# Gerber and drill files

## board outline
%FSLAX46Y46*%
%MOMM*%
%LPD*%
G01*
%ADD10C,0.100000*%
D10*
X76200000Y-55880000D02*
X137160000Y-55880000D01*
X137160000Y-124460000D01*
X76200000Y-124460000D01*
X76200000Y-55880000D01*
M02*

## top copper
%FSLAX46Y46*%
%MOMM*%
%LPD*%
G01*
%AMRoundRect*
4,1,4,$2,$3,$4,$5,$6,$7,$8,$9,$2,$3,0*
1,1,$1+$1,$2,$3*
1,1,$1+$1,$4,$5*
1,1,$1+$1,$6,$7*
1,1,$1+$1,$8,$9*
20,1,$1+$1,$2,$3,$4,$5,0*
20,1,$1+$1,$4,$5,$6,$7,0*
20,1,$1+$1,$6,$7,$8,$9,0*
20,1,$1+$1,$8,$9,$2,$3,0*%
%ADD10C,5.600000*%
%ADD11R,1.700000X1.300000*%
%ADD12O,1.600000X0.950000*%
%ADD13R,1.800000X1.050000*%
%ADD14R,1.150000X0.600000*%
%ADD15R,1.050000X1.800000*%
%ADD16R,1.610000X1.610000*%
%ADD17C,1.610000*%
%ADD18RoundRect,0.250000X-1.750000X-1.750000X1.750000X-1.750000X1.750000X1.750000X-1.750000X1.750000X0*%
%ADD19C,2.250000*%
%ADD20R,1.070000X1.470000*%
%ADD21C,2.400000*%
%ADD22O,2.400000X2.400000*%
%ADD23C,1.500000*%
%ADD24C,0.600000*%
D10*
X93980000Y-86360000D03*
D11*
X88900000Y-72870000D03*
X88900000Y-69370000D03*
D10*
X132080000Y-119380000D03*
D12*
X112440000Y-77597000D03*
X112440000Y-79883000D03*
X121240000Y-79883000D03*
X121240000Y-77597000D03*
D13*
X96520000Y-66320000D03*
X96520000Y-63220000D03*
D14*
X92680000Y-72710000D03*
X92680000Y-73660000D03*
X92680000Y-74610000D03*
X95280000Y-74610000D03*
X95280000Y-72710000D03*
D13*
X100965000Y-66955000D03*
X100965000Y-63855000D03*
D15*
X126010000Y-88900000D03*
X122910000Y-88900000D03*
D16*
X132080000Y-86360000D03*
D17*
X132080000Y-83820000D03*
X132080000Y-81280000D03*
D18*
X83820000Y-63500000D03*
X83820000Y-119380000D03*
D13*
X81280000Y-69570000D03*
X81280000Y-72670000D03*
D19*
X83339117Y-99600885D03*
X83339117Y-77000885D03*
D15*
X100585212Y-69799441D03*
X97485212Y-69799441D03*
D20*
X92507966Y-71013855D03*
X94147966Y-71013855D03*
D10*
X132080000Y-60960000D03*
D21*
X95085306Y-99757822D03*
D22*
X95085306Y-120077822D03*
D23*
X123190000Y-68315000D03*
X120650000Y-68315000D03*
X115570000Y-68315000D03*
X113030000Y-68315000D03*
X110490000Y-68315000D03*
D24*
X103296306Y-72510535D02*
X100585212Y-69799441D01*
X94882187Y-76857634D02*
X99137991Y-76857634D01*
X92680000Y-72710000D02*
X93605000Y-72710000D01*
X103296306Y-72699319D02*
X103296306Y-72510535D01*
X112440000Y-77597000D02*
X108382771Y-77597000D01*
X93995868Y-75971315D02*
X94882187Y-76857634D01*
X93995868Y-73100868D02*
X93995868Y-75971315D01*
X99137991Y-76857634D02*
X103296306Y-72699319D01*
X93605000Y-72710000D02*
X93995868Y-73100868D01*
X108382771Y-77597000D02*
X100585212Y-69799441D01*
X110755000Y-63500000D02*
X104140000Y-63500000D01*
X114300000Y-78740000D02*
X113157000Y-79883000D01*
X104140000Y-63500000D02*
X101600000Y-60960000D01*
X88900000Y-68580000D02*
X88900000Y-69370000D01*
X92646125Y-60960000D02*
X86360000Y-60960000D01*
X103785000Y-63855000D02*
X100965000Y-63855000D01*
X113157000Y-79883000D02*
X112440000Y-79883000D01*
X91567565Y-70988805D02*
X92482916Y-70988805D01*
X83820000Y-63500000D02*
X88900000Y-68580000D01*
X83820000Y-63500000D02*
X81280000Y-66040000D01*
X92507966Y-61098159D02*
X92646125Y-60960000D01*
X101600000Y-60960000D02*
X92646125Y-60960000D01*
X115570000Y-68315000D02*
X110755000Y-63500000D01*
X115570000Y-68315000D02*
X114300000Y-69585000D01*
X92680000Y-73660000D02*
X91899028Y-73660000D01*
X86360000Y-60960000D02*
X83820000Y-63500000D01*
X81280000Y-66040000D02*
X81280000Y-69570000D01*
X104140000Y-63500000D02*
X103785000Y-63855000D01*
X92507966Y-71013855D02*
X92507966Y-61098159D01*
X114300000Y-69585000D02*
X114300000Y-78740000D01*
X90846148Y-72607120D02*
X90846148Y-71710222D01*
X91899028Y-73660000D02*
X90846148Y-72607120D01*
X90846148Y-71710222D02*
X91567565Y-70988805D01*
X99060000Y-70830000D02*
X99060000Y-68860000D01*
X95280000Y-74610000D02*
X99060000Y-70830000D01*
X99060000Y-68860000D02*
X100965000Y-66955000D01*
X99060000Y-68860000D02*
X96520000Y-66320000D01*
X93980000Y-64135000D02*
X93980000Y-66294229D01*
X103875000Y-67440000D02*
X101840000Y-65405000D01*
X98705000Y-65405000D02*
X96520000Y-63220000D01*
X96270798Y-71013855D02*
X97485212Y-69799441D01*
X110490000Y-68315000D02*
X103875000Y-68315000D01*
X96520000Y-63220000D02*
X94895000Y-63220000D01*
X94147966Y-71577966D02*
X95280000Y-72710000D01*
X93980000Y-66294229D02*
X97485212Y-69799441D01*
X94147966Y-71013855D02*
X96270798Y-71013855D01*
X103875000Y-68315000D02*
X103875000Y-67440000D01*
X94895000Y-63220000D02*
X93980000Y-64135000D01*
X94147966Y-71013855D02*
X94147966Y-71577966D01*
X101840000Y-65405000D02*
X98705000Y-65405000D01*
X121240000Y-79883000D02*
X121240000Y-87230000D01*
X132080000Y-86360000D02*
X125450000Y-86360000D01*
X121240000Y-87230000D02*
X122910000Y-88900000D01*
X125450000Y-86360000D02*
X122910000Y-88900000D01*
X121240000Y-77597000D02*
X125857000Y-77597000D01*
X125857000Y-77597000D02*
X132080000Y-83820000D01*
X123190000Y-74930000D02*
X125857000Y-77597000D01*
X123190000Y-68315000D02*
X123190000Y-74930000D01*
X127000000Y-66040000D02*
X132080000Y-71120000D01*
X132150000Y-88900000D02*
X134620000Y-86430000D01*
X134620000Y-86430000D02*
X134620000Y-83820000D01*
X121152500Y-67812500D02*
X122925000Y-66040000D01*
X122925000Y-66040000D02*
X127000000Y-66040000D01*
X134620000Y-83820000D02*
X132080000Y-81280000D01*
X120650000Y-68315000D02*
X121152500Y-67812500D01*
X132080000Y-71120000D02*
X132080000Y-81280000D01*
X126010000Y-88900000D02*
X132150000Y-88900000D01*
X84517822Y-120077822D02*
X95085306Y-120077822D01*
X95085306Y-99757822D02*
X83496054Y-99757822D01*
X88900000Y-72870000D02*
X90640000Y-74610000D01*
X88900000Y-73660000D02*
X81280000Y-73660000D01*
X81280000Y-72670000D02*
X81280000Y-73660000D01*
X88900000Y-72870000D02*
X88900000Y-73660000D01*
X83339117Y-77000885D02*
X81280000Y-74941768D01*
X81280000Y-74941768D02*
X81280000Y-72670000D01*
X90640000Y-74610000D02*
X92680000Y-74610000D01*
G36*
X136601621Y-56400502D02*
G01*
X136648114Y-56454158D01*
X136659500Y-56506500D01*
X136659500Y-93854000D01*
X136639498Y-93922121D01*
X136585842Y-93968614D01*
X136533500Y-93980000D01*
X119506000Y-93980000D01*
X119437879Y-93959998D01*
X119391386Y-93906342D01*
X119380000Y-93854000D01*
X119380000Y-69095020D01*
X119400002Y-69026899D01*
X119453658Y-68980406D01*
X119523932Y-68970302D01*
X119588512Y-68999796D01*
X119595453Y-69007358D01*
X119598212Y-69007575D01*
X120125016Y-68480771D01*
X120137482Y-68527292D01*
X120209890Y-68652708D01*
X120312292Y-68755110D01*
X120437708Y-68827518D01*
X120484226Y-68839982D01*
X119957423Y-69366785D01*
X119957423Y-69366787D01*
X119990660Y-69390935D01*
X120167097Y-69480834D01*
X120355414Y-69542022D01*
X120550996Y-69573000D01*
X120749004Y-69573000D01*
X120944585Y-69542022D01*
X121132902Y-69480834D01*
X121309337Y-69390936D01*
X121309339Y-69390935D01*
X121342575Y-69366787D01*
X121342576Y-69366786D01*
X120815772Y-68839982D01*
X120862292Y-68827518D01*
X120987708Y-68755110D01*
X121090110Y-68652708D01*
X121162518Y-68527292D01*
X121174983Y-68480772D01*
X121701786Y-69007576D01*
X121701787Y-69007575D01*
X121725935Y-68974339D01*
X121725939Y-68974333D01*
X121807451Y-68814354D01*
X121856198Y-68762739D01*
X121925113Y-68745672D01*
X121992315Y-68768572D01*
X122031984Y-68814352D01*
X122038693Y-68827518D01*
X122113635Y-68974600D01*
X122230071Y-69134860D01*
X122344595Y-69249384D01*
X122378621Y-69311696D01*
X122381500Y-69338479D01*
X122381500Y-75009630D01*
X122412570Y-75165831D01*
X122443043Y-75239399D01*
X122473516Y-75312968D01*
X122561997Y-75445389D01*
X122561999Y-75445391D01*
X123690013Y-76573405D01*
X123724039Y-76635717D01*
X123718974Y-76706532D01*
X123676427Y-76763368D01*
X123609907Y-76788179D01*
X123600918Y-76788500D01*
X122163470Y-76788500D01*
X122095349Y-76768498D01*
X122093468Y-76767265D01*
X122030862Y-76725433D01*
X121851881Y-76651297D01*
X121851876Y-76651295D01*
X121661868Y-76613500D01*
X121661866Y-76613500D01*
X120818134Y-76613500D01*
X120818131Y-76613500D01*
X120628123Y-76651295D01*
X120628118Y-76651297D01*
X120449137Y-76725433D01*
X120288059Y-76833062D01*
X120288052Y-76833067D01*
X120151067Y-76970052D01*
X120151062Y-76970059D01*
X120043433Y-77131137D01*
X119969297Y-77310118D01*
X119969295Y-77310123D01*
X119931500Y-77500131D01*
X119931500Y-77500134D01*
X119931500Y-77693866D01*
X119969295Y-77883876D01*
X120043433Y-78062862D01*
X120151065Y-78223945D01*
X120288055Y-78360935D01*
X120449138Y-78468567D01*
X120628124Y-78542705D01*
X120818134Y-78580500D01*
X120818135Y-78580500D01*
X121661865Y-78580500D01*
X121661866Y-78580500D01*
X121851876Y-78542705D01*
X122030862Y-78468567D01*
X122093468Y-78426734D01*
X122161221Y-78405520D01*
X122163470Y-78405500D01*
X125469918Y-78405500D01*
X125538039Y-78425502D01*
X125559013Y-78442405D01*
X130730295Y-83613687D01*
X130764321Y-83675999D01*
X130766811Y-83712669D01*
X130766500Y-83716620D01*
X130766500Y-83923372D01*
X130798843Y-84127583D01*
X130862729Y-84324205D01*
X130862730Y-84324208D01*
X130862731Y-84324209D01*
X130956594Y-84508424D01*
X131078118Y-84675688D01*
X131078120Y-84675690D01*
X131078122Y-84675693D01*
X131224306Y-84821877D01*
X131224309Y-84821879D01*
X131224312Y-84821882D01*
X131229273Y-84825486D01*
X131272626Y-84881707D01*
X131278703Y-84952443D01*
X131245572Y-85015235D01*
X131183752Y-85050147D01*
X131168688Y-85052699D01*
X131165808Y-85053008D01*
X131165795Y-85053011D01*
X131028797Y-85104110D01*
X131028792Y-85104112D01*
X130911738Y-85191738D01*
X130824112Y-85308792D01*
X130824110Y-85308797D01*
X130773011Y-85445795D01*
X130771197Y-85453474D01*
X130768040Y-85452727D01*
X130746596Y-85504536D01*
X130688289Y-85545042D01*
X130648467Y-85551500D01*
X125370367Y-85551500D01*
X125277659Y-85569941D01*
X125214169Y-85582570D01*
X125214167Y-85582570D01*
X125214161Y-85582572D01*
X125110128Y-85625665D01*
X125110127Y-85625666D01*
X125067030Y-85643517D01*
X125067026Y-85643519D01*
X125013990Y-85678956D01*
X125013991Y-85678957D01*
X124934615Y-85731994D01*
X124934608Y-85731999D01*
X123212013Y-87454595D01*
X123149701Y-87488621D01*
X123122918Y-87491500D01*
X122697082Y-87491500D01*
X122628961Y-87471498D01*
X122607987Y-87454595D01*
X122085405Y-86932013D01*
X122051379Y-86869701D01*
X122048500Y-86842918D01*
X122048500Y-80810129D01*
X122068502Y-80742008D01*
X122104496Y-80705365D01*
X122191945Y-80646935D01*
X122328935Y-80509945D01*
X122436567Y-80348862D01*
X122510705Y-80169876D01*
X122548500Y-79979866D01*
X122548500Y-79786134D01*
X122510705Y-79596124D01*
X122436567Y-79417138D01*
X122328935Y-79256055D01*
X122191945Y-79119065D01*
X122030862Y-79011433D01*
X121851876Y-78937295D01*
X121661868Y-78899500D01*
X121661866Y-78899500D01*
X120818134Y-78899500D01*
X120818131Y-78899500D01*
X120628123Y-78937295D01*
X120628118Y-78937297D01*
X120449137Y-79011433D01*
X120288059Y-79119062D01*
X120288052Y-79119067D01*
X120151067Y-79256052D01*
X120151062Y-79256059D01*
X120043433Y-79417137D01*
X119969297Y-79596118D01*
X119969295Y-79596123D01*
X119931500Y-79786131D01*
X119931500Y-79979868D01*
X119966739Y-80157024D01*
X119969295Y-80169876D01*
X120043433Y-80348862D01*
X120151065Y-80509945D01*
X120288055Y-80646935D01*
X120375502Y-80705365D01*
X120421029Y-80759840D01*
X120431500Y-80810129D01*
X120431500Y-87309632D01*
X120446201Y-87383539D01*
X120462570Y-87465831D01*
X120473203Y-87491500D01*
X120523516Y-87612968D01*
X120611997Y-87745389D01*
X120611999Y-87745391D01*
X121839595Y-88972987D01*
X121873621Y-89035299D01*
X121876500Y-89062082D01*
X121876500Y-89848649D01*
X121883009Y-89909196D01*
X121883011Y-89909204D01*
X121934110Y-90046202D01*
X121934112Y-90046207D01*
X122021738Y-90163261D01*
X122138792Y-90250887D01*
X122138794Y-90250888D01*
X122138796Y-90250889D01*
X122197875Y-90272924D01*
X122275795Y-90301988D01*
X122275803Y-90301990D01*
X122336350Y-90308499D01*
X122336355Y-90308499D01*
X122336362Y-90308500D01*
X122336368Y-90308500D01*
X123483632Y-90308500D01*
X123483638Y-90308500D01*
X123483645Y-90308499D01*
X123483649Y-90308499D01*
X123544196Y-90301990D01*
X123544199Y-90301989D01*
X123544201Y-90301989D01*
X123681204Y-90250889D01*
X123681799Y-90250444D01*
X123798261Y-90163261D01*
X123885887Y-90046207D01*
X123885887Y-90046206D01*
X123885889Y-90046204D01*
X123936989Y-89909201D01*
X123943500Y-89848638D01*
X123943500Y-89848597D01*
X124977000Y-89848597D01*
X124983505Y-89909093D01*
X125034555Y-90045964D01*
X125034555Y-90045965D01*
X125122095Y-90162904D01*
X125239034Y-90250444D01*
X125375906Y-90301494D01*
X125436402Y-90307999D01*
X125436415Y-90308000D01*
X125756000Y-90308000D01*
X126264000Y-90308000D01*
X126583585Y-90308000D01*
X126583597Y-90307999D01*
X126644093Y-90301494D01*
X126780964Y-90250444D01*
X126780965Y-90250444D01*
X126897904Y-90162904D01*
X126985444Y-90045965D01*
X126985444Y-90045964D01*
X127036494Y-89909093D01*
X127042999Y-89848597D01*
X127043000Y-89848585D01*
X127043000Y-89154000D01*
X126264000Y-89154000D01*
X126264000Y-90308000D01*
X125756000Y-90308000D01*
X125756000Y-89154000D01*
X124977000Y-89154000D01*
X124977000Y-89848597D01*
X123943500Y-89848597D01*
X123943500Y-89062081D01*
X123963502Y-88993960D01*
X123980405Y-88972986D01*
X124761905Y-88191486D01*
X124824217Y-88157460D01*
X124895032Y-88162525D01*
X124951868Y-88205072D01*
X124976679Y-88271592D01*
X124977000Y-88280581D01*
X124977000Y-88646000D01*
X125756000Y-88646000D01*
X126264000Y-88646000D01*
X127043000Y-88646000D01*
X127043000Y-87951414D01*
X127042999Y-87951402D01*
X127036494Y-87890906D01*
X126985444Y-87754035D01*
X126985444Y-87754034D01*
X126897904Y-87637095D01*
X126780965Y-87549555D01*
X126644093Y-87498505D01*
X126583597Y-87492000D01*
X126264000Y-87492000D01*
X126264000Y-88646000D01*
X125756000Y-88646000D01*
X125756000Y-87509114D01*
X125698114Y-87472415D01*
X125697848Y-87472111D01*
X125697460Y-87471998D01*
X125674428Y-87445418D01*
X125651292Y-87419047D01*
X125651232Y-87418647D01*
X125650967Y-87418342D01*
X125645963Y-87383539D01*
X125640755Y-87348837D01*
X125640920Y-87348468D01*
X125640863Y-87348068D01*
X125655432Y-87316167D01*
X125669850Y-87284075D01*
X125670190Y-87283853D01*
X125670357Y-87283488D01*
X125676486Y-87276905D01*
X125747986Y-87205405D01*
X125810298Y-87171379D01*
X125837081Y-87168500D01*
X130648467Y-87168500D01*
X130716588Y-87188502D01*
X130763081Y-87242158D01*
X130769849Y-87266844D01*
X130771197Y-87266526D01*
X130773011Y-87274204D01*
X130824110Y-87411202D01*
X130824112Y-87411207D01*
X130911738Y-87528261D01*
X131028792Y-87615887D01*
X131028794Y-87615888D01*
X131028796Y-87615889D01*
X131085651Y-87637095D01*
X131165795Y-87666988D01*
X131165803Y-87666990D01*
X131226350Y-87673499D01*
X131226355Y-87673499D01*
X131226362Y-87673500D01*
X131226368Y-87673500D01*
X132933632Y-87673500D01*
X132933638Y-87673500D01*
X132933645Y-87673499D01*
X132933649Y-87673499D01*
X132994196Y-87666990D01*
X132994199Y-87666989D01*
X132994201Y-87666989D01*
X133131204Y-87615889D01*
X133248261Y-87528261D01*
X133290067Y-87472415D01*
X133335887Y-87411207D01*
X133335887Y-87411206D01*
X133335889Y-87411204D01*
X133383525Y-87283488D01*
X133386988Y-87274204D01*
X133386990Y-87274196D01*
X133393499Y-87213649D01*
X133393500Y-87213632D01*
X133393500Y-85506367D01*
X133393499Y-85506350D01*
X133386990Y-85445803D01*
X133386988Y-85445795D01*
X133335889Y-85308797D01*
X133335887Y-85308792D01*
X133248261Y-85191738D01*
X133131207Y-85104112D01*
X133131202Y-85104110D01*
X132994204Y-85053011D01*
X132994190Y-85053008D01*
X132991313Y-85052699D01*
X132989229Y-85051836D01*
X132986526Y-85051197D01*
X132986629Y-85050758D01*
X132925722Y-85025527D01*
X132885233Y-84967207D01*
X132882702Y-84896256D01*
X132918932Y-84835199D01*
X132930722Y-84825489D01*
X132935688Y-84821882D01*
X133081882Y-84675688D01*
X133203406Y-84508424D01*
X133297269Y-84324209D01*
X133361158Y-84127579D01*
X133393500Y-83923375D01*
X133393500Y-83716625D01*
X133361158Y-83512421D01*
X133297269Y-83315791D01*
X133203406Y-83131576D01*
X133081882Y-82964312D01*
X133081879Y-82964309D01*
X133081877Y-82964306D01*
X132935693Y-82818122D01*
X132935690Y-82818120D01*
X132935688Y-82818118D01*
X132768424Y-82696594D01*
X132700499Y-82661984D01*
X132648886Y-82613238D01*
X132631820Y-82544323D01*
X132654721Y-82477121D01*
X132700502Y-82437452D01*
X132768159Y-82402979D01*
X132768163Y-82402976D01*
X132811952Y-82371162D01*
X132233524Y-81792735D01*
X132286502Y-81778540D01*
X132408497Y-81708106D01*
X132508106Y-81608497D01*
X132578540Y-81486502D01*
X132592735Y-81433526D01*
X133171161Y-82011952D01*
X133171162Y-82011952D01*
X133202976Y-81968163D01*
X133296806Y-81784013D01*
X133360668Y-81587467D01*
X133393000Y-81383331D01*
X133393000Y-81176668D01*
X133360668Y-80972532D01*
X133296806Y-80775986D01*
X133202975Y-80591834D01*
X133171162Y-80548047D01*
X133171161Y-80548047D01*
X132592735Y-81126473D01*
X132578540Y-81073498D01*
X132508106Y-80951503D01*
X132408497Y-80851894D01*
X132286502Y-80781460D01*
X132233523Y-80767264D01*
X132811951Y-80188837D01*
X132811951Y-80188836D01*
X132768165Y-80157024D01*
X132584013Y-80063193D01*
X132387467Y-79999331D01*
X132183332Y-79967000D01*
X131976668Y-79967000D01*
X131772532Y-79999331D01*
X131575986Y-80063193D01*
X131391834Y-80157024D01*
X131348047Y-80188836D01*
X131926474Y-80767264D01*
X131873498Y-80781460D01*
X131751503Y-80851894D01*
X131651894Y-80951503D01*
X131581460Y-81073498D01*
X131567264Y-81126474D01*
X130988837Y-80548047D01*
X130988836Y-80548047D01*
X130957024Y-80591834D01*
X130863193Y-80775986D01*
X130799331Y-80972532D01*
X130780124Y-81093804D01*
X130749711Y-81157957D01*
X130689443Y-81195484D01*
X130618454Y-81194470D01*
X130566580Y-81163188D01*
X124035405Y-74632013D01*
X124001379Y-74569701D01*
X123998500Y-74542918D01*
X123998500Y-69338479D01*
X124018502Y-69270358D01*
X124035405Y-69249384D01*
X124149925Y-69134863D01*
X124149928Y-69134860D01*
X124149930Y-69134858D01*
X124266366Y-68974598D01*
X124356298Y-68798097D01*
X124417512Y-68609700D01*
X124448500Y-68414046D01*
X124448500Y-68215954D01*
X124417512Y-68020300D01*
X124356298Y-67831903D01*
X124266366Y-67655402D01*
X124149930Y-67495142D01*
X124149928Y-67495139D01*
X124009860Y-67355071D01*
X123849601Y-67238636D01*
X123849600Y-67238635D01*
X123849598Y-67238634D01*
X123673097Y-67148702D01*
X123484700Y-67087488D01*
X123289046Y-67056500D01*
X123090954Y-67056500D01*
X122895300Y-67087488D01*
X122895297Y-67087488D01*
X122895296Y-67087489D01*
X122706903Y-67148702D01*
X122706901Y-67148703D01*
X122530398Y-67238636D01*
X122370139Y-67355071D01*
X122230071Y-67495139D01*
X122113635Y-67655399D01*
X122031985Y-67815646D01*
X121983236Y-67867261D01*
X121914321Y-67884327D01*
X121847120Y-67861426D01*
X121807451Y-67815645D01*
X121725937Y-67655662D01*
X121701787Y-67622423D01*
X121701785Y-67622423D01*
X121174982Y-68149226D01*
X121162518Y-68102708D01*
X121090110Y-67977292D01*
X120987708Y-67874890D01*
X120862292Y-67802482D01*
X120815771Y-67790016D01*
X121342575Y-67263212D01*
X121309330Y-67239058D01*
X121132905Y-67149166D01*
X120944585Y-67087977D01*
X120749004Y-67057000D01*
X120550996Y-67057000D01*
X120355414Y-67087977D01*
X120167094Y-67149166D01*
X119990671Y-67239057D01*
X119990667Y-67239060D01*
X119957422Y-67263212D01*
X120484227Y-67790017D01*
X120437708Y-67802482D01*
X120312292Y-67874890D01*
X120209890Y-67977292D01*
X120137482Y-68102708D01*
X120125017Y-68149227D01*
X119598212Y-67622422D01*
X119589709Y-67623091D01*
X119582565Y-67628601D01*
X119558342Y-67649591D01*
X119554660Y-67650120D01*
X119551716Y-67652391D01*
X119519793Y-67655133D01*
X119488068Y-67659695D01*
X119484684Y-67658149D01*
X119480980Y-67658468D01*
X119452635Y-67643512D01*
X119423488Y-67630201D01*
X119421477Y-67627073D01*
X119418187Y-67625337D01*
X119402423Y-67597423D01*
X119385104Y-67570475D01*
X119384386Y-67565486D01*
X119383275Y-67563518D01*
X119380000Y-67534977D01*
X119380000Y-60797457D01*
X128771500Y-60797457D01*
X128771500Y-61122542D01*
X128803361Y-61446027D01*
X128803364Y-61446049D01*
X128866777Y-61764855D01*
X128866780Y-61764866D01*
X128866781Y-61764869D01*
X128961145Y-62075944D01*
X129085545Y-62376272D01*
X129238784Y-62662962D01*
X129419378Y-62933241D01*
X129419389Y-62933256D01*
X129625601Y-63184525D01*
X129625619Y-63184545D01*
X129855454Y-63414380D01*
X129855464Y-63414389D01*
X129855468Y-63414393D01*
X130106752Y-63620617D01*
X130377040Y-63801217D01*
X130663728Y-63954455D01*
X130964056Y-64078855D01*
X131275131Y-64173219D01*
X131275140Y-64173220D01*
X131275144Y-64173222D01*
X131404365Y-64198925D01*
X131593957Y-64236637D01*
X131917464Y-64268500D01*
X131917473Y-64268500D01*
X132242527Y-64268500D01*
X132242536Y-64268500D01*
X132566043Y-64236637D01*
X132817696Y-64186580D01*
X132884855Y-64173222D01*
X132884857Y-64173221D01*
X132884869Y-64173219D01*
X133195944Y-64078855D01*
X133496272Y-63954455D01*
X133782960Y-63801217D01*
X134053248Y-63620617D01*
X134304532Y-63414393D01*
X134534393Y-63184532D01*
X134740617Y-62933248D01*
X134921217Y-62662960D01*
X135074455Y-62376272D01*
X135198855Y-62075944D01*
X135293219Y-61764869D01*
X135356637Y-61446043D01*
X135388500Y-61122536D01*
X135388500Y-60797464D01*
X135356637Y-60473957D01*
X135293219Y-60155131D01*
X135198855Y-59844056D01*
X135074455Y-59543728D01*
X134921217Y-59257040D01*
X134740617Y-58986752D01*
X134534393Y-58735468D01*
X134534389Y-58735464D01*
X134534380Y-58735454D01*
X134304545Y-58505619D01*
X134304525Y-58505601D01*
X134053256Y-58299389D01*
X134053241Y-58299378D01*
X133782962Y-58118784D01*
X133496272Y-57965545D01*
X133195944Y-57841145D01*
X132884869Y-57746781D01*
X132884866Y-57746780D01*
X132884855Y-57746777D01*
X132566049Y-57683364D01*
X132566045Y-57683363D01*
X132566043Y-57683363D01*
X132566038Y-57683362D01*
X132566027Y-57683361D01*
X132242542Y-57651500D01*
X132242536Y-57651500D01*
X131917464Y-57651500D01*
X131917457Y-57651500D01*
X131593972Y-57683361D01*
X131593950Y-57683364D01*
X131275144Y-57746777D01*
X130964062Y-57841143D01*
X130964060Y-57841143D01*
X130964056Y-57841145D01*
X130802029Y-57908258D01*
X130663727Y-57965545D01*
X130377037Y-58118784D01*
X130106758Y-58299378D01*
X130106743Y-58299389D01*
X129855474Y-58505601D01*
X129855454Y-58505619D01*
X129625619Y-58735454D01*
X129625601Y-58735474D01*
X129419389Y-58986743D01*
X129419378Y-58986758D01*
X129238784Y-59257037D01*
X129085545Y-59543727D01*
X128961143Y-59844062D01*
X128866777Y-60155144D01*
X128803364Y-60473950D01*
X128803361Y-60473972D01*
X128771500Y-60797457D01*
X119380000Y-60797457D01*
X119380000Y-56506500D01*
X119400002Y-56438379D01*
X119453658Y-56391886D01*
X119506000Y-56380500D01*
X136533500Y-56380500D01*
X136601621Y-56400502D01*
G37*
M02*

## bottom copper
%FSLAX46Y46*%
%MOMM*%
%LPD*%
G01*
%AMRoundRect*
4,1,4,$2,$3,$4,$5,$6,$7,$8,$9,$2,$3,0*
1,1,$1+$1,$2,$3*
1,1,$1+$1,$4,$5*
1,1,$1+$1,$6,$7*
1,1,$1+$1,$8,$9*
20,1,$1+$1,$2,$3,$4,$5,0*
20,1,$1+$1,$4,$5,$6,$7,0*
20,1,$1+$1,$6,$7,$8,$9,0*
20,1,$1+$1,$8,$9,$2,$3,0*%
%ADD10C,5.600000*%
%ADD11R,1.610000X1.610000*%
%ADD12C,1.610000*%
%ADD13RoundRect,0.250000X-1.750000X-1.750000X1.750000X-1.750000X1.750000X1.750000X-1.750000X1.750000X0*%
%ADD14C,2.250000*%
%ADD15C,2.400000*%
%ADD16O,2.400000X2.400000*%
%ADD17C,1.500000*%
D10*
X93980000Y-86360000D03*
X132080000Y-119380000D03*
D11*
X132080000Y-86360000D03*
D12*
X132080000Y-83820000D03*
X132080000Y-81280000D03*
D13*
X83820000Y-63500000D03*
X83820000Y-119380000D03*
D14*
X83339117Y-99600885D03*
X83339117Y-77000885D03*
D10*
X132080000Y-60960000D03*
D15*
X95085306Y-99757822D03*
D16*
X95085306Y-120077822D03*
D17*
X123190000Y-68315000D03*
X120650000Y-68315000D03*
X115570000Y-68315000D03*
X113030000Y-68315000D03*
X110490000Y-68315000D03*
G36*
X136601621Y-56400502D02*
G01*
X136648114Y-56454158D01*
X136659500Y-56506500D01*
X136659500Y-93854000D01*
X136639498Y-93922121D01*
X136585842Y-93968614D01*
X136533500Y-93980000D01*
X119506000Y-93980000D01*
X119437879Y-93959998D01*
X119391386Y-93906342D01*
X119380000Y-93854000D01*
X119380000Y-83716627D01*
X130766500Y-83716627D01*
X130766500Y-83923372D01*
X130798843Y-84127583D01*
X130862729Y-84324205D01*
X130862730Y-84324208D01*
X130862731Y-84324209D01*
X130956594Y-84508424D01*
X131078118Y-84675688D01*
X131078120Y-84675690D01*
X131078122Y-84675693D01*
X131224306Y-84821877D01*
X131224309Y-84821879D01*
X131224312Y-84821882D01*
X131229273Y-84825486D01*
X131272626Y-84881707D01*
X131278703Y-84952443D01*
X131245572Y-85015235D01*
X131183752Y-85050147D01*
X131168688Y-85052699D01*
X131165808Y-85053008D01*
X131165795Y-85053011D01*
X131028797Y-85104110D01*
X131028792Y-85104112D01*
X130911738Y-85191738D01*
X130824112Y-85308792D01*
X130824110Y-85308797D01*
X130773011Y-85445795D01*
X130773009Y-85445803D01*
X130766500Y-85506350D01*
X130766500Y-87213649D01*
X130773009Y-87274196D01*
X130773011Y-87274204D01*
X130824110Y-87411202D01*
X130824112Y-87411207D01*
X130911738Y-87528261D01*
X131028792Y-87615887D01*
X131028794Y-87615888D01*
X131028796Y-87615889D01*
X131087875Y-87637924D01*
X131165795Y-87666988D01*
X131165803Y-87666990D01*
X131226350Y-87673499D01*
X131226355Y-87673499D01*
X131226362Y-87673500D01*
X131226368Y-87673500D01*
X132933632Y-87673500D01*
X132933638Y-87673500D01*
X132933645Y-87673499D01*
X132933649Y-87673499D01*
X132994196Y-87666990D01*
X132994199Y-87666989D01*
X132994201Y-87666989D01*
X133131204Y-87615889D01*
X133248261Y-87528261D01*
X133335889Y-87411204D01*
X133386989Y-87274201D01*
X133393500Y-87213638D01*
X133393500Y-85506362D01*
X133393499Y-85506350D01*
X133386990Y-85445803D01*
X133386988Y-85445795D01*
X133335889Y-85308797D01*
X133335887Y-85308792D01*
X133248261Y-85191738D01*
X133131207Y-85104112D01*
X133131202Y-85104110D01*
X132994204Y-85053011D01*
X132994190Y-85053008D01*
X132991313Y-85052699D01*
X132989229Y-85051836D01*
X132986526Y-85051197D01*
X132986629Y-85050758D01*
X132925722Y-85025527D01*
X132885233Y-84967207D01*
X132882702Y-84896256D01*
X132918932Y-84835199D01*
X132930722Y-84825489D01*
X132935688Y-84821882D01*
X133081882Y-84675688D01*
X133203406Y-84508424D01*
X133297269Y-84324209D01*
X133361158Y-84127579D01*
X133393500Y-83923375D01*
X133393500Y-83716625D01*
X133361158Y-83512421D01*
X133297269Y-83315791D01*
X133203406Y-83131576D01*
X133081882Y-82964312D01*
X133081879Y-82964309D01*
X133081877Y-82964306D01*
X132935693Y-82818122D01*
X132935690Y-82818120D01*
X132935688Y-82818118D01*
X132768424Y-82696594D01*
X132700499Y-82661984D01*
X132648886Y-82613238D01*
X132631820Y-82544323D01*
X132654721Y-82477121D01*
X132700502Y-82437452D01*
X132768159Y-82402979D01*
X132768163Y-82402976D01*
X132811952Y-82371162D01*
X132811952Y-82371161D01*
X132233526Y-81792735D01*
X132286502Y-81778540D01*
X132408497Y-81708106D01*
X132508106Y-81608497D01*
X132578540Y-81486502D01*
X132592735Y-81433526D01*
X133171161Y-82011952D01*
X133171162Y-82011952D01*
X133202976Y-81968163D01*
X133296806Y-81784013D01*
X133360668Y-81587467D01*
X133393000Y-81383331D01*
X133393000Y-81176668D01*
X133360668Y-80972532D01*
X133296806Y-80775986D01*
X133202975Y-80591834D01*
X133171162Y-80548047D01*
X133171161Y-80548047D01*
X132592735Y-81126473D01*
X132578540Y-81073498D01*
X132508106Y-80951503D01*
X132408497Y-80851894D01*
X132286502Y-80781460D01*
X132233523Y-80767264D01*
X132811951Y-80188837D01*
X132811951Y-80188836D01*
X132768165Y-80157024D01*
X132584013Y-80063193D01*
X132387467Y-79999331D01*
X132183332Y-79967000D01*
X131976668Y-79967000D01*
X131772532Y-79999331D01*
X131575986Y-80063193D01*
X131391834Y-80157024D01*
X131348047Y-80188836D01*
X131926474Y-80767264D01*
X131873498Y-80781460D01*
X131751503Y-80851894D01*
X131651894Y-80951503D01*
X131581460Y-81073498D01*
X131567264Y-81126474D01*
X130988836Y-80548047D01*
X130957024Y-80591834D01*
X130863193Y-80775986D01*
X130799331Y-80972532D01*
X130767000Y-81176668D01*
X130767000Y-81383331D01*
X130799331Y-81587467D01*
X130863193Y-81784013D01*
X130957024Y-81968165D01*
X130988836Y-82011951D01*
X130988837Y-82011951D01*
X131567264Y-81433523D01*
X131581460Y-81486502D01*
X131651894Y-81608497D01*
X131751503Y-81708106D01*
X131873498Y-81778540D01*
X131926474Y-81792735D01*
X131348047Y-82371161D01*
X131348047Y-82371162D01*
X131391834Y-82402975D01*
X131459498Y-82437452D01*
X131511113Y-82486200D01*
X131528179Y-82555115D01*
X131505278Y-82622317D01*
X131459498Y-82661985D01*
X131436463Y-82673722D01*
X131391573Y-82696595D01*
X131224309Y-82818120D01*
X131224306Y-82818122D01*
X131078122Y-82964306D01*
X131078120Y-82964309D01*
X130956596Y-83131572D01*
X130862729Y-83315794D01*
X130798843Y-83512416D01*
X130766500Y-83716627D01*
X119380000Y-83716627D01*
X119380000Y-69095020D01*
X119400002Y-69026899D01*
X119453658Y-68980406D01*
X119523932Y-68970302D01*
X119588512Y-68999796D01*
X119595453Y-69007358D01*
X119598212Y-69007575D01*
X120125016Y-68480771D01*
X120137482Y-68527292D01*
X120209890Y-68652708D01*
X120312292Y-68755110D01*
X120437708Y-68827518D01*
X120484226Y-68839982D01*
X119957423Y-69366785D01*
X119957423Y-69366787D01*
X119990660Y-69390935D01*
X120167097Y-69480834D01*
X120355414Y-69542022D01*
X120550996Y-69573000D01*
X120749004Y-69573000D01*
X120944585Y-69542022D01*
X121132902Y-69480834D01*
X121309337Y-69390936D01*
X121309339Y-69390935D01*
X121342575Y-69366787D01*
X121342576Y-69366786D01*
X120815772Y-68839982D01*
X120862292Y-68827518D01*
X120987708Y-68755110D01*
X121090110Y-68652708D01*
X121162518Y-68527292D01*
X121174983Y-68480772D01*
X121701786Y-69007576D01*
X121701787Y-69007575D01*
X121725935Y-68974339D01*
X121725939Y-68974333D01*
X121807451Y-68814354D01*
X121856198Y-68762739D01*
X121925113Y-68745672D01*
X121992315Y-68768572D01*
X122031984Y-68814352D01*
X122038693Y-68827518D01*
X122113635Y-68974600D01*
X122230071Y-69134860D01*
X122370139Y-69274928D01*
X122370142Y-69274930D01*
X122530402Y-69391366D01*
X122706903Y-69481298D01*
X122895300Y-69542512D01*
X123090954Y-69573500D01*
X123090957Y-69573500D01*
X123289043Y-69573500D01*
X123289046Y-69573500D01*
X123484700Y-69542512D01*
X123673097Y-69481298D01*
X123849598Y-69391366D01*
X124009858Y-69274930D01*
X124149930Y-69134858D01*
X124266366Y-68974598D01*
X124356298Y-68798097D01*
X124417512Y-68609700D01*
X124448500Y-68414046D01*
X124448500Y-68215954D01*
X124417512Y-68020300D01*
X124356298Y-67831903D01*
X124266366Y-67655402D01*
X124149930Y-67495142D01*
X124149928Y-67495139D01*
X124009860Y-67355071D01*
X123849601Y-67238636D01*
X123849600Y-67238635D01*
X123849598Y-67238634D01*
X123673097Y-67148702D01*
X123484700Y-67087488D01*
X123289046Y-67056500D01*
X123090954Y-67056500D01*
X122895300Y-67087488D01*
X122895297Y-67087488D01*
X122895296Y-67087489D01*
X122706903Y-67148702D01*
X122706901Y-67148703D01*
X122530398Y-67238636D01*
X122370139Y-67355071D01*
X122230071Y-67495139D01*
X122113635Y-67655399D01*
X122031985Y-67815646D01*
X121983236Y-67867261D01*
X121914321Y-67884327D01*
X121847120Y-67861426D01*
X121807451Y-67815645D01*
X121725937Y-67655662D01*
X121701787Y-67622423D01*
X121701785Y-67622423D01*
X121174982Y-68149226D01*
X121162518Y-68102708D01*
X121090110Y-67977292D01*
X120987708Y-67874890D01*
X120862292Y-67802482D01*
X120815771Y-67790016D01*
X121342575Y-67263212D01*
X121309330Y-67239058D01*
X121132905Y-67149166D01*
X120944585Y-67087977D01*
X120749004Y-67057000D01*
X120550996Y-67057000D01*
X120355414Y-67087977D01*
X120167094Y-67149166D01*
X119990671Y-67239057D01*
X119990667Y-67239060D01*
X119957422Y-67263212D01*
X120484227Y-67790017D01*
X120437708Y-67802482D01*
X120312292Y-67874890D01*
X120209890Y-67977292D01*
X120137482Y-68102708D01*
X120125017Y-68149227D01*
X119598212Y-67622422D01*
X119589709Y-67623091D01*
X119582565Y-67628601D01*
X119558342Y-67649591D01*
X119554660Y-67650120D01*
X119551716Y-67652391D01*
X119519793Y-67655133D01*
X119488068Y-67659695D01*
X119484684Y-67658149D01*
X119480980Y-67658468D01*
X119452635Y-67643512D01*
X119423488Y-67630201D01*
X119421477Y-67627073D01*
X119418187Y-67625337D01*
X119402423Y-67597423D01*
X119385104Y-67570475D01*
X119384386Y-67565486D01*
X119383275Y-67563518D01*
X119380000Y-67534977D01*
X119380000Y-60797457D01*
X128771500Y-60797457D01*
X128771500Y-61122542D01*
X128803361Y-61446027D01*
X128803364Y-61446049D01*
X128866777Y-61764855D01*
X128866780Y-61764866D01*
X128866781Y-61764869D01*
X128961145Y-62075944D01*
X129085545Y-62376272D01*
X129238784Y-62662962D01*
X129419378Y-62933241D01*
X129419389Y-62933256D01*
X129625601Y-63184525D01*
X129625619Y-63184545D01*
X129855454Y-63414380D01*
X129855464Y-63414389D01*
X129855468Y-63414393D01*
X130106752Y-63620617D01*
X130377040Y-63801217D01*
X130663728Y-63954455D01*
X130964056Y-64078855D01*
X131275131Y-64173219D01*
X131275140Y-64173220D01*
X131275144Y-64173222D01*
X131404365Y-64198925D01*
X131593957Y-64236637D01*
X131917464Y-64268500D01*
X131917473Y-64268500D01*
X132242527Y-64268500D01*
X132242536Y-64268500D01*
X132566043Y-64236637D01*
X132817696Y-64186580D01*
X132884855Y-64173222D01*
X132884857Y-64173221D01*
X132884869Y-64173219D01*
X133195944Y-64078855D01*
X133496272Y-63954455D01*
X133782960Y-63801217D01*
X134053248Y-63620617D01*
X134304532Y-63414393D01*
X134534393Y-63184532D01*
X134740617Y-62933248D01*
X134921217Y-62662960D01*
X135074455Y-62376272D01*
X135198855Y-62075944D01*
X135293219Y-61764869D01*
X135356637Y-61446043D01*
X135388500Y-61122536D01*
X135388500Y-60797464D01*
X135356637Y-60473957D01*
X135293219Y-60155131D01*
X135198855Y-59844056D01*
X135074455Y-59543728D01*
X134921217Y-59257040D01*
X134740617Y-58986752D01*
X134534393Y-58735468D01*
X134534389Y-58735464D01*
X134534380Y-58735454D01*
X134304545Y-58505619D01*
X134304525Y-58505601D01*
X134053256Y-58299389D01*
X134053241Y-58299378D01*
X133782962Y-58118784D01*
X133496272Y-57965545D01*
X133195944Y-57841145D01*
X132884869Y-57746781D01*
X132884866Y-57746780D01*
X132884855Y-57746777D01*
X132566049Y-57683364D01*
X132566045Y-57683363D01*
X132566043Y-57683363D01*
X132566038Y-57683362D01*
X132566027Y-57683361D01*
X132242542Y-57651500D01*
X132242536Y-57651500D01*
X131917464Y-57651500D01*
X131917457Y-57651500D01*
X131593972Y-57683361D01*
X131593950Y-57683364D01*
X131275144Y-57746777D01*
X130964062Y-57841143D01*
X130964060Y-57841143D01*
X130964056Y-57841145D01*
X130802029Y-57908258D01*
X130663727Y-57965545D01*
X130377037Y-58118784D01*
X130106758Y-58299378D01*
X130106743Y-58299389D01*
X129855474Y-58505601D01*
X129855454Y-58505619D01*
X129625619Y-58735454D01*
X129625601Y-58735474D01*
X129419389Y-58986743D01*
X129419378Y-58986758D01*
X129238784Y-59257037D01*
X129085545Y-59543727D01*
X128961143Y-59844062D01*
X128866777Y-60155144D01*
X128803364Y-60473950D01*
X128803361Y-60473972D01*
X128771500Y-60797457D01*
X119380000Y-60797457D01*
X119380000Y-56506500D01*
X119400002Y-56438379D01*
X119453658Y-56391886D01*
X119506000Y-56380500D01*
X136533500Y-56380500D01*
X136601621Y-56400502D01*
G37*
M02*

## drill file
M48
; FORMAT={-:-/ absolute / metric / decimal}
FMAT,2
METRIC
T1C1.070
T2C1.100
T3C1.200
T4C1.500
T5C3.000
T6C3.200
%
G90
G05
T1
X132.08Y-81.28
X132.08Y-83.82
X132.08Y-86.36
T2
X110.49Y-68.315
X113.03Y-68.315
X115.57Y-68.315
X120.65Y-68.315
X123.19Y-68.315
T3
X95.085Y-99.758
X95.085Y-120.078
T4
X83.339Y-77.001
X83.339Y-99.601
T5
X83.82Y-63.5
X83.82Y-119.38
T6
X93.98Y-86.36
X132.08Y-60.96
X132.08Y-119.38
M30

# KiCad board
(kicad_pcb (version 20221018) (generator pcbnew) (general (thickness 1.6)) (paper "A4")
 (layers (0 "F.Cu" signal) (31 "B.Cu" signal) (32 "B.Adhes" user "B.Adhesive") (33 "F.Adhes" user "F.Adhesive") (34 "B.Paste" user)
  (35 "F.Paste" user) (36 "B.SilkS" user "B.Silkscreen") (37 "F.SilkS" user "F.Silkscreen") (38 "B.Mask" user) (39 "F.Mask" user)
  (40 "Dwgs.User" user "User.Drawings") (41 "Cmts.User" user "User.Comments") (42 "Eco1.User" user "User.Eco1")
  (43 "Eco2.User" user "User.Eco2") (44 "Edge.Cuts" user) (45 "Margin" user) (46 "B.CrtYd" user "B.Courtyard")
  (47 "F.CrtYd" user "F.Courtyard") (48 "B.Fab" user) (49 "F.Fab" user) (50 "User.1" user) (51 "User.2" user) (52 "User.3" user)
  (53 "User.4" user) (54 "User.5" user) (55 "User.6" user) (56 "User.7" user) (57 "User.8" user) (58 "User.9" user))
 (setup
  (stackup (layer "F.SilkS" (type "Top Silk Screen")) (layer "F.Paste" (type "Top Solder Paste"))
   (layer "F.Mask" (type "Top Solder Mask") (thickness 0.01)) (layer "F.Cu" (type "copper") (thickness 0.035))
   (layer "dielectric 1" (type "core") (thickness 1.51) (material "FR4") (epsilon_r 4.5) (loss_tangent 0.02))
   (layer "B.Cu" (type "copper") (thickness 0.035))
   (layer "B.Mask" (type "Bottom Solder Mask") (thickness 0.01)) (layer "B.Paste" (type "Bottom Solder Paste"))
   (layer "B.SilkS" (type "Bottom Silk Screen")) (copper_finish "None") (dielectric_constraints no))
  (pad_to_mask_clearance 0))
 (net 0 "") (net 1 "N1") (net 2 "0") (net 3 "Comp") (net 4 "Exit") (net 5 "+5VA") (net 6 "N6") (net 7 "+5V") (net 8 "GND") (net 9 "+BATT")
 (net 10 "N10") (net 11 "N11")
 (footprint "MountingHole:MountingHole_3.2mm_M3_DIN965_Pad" (layer "F.Cu") (at 93.98 86.36)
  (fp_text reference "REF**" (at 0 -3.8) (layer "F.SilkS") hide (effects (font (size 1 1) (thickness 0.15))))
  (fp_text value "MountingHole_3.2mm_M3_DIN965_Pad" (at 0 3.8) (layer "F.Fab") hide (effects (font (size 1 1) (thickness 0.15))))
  (pad "1" thru_hole circle (at 0 0) (size 5.6 5.6) (drill 3.2) (layers "*.Cu" "*.Mask")))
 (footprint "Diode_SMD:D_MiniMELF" (layer "F.Cu") (at 88.9 71.12 90)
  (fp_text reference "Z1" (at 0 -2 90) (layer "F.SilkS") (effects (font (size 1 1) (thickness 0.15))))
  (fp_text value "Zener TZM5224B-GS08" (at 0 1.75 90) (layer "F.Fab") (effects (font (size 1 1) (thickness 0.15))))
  (pad "1" smd rect (at -1.75 0 90) (size 1.3 1.7) (layers "F.Cu" "F.Paste" "F.Mask") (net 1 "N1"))
  (pad "2" smd rect (at 1.75 0 90) (size 1.3 1.7) (layers "F.Cu" "F.Paste" "F.Mask") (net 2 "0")))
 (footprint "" (layer "F.Cu") (at 132.08 119.38)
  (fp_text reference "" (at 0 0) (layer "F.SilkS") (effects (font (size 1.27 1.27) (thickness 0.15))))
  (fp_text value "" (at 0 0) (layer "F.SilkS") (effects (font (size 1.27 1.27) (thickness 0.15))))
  (pad "1" thru_hole circle (at 0 0) (size 5.6 5.6) (drill 3.2) (layers "*.Cu" "*.Mask")))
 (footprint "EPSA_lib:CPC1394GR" (layer "F.Cu") (at 116.84 78.74 -90)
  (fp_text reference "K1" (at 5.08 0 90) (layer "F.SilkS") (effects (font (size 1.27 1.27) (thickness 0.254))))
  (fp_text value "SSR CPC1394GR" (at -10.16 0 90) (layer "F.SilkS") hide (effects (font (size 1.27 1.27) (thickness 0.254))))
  (pad "1" smd oval (at -1.143 4.4 270) (size 0.95 1.6) (layers "F.Cu" "F.Paste" "F.Mask") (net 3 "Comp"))
  (pad "2" smd oval (at 1.143 4.4 270) (size 0.95 1.6) (layers "F.Cu" "F.Paste" "F.Mask") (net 2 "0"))
  (pad "3" smd oval (at 1.143 -4.4 270) (size 0.95 1.6) (layers "F.Cu" "F.Paste" "F.Mask") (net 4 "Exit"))
  (pad "4" smd oval (at -1.143 -4.4 270) (size 0.95 1.6) (layers "F.Cu" "F.Paste" "F.Mask") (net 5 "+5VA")))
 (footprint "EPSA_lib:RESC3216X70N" (layer "F.Cu") (at 96.52 64.77 90)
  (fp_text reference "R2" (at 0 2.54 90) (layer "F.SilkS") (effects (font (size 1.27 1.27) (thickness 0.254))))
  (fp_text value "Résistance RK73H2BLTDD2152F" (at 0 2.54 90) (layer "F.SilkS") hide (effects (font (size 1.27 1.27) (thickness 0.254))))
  (pad "1" smd rect (at -1.55 0 90) (size 1.05 1.8) (layers "F.Cu" "F.Paste" "F.Mask") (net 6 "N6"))
  (pad "2" smd rect (at 1.55 0 90) (size 1.05 1.8) (layers "F.Cu" "F.Paste" "F.Mask") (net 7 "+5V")))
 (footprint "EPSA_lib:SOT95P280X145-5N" (layer "F.Cu") (at 93.98 73.66)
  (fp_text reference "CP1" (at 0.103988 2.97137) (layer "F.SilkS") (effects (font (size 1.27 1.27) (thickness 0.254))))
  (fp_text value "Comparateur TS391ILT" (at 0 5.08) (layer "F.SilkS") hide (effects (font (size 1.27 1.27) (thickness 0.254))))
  (pad "1" smd rect (at -1.3 -0.95 90) (size 0.6 1.15) (layers "F.Cu" "F.Paste" "F.Mask") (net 3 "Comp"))
  (pad "2" smd rect (at -1.3 0 90) (size 0.6 1.15) (layers "F.Cu" "F.Paste" "F.Mask") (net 2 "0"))
  (pad "3" smd rect (at -1.3 0.95 90) (size 0.6 1.15) (layers "F.Cu" "F.Paste" "F.Mask") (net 1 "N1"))
  (pad "4" smd rect (at 1.3 0.95 90) (size 0.6 1.15) (layers "F.Cu" "F.Paste" "F.Mask") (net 6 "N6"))
  (pad "5" smd rect (at 1.3 -0.95 90) (size 0.6 1.15) (layers "F.Cu" "F.Paste" "F.Mask") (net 7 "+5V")))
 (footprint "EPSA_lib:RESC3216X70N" (layer "F.Cu") (at 100.965 65.405 90)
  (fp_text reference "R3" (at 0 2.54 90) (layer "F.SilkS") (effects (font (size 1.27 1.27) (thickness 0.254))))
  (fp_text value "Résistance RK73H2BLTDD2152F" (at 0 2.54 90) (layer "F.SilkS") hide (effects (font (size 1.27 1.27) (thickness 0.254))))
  (pad "1" smd rect (at -1.55 0 90) (size 1.05 1.8) (layers "F.Cu" "F.Paste" "F.Mask") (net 6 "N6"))
  (pad "2" smd rect (at 1.55 0 90) (size 1.05 1.8) (layers "F.Cu" "F.Paste" "F.Mask") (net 2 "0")))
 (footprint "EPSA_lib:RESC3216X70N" (layer "F.Cu") (at 124.46 88.9 180)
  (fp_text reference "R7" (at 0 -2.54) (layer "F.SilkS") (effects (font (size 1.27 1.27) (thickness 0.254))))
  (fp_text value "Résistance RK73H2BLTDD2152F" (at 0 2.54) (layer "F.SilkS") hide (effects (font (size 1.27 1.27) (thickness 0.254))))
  (pad "1" smd rect (at -1.55 0 180) (size 1.05 1.8) (layers "F.Cu" "F.Paste" "F.Mask") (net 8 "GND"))
  (pad "2" smd rect (at 1.55 0 180) (size 1.05 1.8) (layers "F.Cu" "F.Paste" "F.Mask") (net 4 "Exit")))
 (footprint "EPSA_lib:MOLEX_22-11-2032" (layer "F.Cu") (at 132.08 86.36 90)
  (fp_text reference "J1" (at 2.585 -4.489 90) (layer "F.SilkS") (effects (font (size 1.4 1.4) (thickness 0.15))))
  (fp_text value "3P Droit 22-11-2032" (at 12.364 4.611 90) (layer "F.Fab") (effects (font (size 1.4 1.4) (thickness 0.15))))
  (pad "1" thru_hole rect (at 0 0 90) (size 1.61 1.61) (drill 1.07) (layers "*.Cu" "*.Mask") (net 4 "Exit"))
  (pad "2" thru_hole circle (at 2.54 0 90) (size 1.61 1.61) (drill 1.07) (layers "*.Cu" "*.Mask") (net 5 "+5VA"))
  (pad "3" thru_hole circle (at 5.08 0 90) (size 1.61 1.61) (drill 1.07) (layers "*.Cu" "*.Mask") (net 8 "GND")))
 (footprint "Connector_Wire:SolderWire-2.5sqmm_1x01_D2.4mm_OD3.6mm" (layer "F.Cu") (at 83.82 63.5)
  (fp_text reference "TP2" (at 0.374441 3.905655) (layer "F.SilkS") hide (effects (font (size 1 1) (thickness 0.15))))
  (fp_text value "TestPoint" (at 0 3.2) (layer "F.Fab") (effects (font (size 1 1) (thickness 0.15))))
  (pad "1" thru_hole roundrect (at 0 0) (size 4 4) (drill 3) (layers "*.Cu" "*.Mask") (roundrect_rratio 0.0625) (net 2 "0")))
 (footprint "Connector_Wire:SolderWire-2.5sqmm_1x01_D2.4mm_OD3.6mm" (layer "F.Cu") (at 83.82 119.38)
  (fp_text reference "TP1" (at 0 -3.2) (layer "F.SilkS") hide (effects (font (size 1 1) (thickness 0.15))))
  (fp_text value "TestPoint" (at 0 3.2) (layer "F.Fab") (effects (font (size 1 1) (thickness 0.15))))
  (pad "1" thru_hole roundrect (at 0 0) (size 4 4) (drill 3) (layers "*.Cu" "*.Mask") (roundrect_rratio 0.0625) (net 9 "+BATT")))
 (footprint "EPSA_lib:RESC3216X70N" (layer "F.Cu") (at 81.28 71.12 -90)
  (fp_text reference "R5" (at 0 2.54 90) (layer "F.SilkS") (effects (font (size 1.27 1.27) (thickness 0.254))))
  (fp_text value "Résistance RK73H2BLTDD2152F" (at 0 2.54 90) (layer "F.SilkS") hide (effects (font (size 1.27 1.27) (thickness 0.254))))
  (pad "1" smd rect (at -1.55 0 270) (size 1.05 1.8) (layers "F.Cu" "F.Paste" "F.Mask") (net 2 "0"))
  (pad "2" smd rect (at 1.55 0 270) (size 1.05 1.8) (layers "F.Cu" "F.Paste" "F.Mask") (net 1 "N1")))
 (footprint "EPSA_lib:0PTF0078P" (layer "F.Cu") (at 83.339117 88.300885 90)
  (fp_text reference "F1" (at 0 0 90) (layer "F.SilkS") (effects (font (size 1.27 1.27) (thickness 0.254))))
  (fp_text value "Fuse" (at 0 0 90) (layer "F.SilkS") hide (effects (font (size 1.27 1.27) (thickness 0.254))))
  (pad "1" thru_hole circle (at -11.3 0 90) (size 2.25 2.25) (drill 1.5) (layers "*.Cu" "*.Mask") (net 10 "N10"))
  (pad "2" thru_hole circle (at 11.3 0 90) (size 2.25 2.25) (drill 1.5) (layers "*.Cu" "*.Mask") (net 1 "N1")))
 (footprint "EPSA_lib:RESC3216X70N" (layer "F.Cu") (at 99.035212 69.799441 180)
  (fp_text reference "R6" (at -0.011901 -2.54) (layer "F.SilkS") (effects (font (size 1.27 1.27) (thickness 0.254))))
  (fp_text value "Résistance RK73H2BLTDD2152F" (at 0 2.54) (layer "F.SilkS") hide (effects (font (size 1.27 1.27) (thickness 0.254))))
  (pad "1" smd rect (at -1.55 0 180) (size 1.05 1.8) (layers "F.Cu" "F.Paste" "F.Mask") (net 3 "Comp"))
  (pad "2" smd rect (at 1.55 0 180) (size 1.05 1.8) (layers "F.Cu" "F.Paste" "F.Mask") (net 7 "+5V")))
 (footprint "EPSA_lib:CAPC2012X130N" (layer "F.Cu") (at 93.327966 71.013855)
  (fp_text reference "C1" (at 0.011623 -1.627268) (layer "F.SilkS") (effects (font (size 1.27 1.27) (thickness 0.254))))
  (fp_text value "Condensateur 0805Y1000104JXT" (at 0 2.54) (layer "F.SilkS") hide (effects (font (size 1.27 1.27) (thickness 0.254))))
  (pad "1" smd rect (at -0.82 0) (size 1.07 1.47) (layers "F.Cu" "F.Paste" "F.Mask") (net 2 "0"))
  (pad "2" smd rect (at 0.82 0) (size 1.07 1.47) (layers "F.Cu" "F.Paste" "F.Mask") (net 7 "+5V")))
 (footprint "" (layer "F.Cu") (at 132.08 60.96)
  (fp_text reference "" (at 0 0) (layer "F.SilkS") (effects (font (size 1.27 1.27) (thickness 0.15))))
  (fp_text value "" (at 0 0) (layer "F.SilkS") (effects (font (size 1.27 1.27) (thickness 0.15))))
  (pad "1" thru_hole circle (at 0 0) (size 5.6 5.6) (drill 3.2) (layers "*.Cu" "*.Mask")))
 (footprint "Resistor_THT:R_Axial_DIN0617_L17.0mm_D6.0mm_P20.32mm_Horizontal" (layer "F.Cu") (at 95.085306 99.757822 -90)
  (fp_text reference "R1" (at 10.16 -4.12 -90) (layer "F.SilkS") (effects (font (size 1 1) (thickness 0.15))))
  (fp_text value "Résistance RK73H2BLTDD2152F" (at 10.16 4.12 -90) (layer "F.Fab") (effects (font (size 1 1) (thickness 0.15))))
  (pad "1" thru_hole circle (at 0 0 270) (size 2.4 2.4) (drill 1.2) (layers "*.Cu" "*.Mask") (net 10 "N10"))
  (pad "2" thru_hole oval (at 20.32 0 270) (size 2.4 2.4) (drill 1.2) (layers "*.Cu" "*.Mask") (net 9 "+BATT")))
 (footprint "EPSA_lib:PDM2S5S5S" (layer "F.Cu") (at 123.19 68.315 180)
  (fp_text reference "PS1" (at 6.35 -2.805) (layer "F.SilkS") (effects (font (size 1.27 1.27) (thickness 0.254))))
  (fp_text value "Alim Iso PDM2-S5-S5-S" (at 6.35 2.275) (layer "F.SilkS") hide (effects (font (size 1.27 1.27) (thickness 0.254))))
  (pad "1" thru_hole circle (at 0 0 180) (size 1.5 1.5) (drill 1.1) (layers "*.Cu" "*.Mask") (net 5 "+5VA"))
  (pad "2" thru_hole circle (at 2.54 0 180) (size 1.5 1.5) (drill 1.1) (layers "*.Cu" "*.Mask") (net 8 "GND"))
  (pad "4" thru_hole circle (at 7.62 0 180) (size 1.5 1.5) (drill 1.1) (layers "*.Cu" "*.Mask") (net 2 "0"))
  (pad "5" thru_hole circle (at 10.16 0 180) (size 1.5 1.5) (drill 1.1) (layers "*.Cu" "*.Mask") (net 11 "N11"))
  (pad "6" thru_hole circle (at 12.7 0 180) (size 1.5 1.5) (drill 1.1) (layers "*.Cu" "*.Mask") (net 7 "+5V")))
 (gr_rect (start 76.2 55.88) (end 137.16 124.46) (stroke (width 0.1) (type solid)) (fill none) (layer "Edge.Cuts"))
 (segment (start 103.296306 72.510535) (end 100.585212 69.799441) (width 0.6) (layer "F.Cu") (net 3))
 (segment (start 94.882187 76.857634) (end 99.137991 76.857634) (width 0.6) (layer "F.Cu") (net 3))
 (segment (start 92.68 72.71) (end 93.605 72.71) (width 0.6) (layer "F.Cu") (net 3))
 (segment (start 103.296306 72.699319) (end 103.296306 72.510535) (width 0.6) (layer "F.Cu") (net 3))
 (segment (start 112.44 77.597) (end 108.382771 77.597) (width 0.6) (layer "F.Cu") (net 3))
 (segment (start 93.995868 75.971315) (end 94.882187 76.857634) (width 0.6) (layer "F.Cu") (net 3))
 (segment (start 93.995868 73.100868) (end 93.995868 75.971315) (width 0.6) (layer "F.Cu") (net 3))
 (segment (start 99.137991 76.857634) (end 103.296306 72.699319) (width 0.6) (layer "F.Cu") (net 3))
 (segment (start 93.605 72.71) (end 93.995868 73.100868) (width 0.6) (layer "F.Cu") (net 3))
 (segment (start 108.382771 77.597) (end 100.585212 69.799441) (width 0.6) (layer "F.Cu") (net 3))
 (segment (start 110.755 63.5) (end 104.14 63.5) (width 0.6) (layer "F.Cu") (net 2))
 (segment (start 114.3 78.74) (end 113.157 79.883) (width 0.6) (layer "F.Cu") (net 2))
 (segment (start 104.14 63.5) (end 101.6 60.96) (width 0.6) (layer "F.Cu") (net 2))
 (segment (start 88.9 68.58) (end 88.9 69.37) (width 0.6) (layer "F.Cu") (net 2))
 (segment (start 92.646125 60.96) (end 86.36 60.96) (width 0.6) (layer "F.Cu") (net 2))
 (segment (start 103.785 63.855) (end 100.965 63.855) (width 0.6) (layer "F.Cu") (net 2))
 (segment (start 113.157 79.883) (end 112.44 79.883) (width 0.6) (layer "F.Cu") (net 2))
 (segment (start 91.567565 70.988805) (end 92.482916 70.988805) (width 0.6) (layer "F.Cu") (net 2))
 (segment (start 83.82 63.5) (end 88.9 68.58) (width 0.6) (layer "F.Cu") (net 2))
 (segment (start 83.82 63.5) (end 81.28 66.04) (width 0.6) (layer "F.Cu") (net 2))
 (segment (start 92.507966 61.098159) (end 92.646125 60.96) (width 0.6) (layer "F.Cu") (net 2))
 (segment (start 101.6 60.96) (end 92.646125 60.96) (width 0.6) (layer "F.Cu") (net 2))
 (segment (start 115.57 68.315) (end 110.755 63.5) (width 0.6) (layer "F.Cu") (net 2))
 (segment (start 115.57 68.315) (end 114.3 69.585) (width 0.6) (layer "F.Cu") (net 2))
 (segment (start 92.68 73.66) (end 91.899028 73.66) (width 0.6) (layer "F.Cu") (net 2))
 (segment (start 86.36 60.96) (end 83.82 63.5) (width 0.6) (layer "F.Cu") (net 2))
 (segment (start 81.28 66.04) (end 81.28 69.57) (width 0.6) (layer "F.Cu") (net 2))
 (segment (start 104.14 63.5) (end 103.785 63.855) (width 0.6) (layer "F.Cu") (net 2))
 (segment (start 92.507966 71.013855) (end 92.507966 61.098159) (width 0.6) (layer "F.Cu") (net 2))
 (segment (start 114.3 69.585) (end 114.3 78.74) (width 0.6) (layer "F.Cu") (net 2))
 (segment (start 90.846148 72.60712) (end 90.846148 71.710222) (width 0.6) (layer "F.Cu") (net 2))
 (segment (start 91.899028 73.66) (end 90.846148 72.60712) (width 0.6) (layer "F.Cu") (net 2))
 (segment (start 90.846148 71.710222) (end 91.567565 70.988805) (width 0.6) (layer "F.Cu") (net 2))
 (segment (start 99.06 70.83) (end 99.06 68.86) (width 0.6) (layer "F.Cu") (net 6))
 (segment (start 95.28 74.61) (end 99.06 70.83) (width 0.6) (layer "F.Cu") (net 6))
 (segment (start 99.06 68.86) (end 100.965 66.955) (width 0.6) (layer "F.Cu") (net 6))
 (segment (start 99.06 68.86) (end 96.52 66.32) (width 0.6) (layer "F.Cu") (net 6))
 (segment (start 93.98 64.135) (end 93.98 66.294229) (width 0.6) (layer "F.Cu") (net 7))
 (segment (start 103.875 67.44) (end 101.84 65.405) (width 0.6) (layer "F.Cu") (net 7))
 (segment (start 98.705 65.405) (end 96.52 63.22) (width 0.6) (layer "F.Cu") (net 7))
 (segment (start 96.270798 71.013855) (end 97.485212 69.799441) (width 0.6) (layer "F.Cu") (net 7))
 (segment (start 110.49 68.315) (end 103.875 68.315) (width 0.6) (layer "F.Cu") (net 7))
 (segment (start 96.52 63.22) (end 94.895 63.22) (width 0.6) (layer "F.Cu") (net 7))
 (segment (start 94.147966 71.577966) (end 95.28 72.71) (width 0.6) (layer "F.Cu") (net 7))
 (segment (start 93.98 66.294229) (end 97.485212 69.799441) (width 0.6) (layer "F.Cu") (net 7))
 (segment (start 94.147966 71.013855) (end 96.270798 71.013855) (width 0.6) (layer "F.Cu") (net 7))
 (segment (start 103.875 68.315) (end 103.875 67.44) (width 0.6) (layer "F.Cu") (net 7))
 (segment (start 94.895 63.22) (end 93.98 64.135) (width 0.6) (layer "F.Cu") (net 7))
 (segment (start 94.147966 71.013855) (end 94.147966 71.577966) (width 0.6) (layer "F.Cu") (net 7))
 (segment (start 101.84 65.405) (end 98.705 65.405) (width 0.6) (layer "F.Cu") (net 7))
 (segment (start 121.24 79.883) (end 121.24 87.23) (width 0.6) (layer "F.Cu") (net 4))
 (segment (start 132.08 86.36) (end 125.45 86.36) (width 0.6) (layer "F.Cu") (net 4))
 (segment (start 121.24 87.23) (end 122.91 88.9) (width 0.6) (layer "F.Cu") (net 4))
 (segment (start 125.45 86.36) (end 122.91 88.9) (width 0.6) (layer "F.Cu") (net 4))
 (segment (start 121.24 77.597) (end 125.857 77.597) (width 0.6) (layer "F.Cu") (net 5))
 (segment (start 125.857 77.597) (end 132.08 83.82) (width 0.6) (layer "F.Cu") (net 5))
 (segment (start 123.19 74.93) (end 125.857 77.597) (width 0.6) (layer "F.Cu") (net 5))
 (segment (start 123.19 68.315) (end 123.19 74.93) (width 0.6) (layer "F.Cu") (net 5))
 (segment (start 127 66.04) (end 132.08 71.12) (width 0.6) (layer "F.Cu") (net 8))
 (segment (start 132.15 88.9) (end 134.62 86.43) (width 0.6) (layer "F.Cu") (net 8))
 (segment (start 134.62 86.43) (end 134.62 83.82) (width 0.6) (layer "F.Cu") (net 8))
 (segment (start 121.1525 67.8125) (end 122.925 66.04) (width 0.6) (layer "F.Cu") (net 8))
 (segment (start 122.925 66.04) (end 127 66.04) (width 0.6) (layer "F.Cu") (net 8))
 (segment (start 134.62 83.82) (end 132.08 81.28) (width 0.6) (layer "F.Cu") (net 8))
 (segment (start 120.65 68.315) (end 121.1525 67.8125) (width 0.6) (layer "F.Cu") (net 8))
 (segment (start 132.08 71.12) (end 132.08 81.28) (width 0.6) (layer "F.Cu") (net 8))
 (segment (start 126.01 88.9) (end 132.15 88.9) (width 0.6) (layer "F.Cu") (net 8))
 (segment (start 84.517822 120.077822) (end 95.085306 120.077822) (width 0.6) (layer "F.Cu") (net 9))
 (segment (start 95.085306 99.757822) (end 83.496054 99.757822) (width 0.6) (layer "F.Cu") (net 10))
 (segment (start 88.9 72.87) (end 90.64 74.61) (width 0.6) (layer "F.Cu") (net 1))
 (segment (start 88.9 73.66) (end 81.28 73.66) (width 0.6) (layer "F.Cu") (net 1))
 (segment (start 81.28 72.67) (end 81.28 73.66) (width 0.6) (layer "F.Cu") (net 1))
 (segment (start 88.9 72.87) (end 88.9 73.66) (width 0.6) (layer "F.Cu") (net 1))
 (segment (start 83.339117 77.000885) (end 81.28 74.941768) (width 0.6) (layer "F.Cu") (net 1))
 (segment (start 81.28 74.941768) (end 81.28 72.67) (width 0.6) (layer "F.Cu") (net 1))
 (segment (start 90.64 74.61) (end 92.68 74.61) (width 0.6) (layer "F.Cu") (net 1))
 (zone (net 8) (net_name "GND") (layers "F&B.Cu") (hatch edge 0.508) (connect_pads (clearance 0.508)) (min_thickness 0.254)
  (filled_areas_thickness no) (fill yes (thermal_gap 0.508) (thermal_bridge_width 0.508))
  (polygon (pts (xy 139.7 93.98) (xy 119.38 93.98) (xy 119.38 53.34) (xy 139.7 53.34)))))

